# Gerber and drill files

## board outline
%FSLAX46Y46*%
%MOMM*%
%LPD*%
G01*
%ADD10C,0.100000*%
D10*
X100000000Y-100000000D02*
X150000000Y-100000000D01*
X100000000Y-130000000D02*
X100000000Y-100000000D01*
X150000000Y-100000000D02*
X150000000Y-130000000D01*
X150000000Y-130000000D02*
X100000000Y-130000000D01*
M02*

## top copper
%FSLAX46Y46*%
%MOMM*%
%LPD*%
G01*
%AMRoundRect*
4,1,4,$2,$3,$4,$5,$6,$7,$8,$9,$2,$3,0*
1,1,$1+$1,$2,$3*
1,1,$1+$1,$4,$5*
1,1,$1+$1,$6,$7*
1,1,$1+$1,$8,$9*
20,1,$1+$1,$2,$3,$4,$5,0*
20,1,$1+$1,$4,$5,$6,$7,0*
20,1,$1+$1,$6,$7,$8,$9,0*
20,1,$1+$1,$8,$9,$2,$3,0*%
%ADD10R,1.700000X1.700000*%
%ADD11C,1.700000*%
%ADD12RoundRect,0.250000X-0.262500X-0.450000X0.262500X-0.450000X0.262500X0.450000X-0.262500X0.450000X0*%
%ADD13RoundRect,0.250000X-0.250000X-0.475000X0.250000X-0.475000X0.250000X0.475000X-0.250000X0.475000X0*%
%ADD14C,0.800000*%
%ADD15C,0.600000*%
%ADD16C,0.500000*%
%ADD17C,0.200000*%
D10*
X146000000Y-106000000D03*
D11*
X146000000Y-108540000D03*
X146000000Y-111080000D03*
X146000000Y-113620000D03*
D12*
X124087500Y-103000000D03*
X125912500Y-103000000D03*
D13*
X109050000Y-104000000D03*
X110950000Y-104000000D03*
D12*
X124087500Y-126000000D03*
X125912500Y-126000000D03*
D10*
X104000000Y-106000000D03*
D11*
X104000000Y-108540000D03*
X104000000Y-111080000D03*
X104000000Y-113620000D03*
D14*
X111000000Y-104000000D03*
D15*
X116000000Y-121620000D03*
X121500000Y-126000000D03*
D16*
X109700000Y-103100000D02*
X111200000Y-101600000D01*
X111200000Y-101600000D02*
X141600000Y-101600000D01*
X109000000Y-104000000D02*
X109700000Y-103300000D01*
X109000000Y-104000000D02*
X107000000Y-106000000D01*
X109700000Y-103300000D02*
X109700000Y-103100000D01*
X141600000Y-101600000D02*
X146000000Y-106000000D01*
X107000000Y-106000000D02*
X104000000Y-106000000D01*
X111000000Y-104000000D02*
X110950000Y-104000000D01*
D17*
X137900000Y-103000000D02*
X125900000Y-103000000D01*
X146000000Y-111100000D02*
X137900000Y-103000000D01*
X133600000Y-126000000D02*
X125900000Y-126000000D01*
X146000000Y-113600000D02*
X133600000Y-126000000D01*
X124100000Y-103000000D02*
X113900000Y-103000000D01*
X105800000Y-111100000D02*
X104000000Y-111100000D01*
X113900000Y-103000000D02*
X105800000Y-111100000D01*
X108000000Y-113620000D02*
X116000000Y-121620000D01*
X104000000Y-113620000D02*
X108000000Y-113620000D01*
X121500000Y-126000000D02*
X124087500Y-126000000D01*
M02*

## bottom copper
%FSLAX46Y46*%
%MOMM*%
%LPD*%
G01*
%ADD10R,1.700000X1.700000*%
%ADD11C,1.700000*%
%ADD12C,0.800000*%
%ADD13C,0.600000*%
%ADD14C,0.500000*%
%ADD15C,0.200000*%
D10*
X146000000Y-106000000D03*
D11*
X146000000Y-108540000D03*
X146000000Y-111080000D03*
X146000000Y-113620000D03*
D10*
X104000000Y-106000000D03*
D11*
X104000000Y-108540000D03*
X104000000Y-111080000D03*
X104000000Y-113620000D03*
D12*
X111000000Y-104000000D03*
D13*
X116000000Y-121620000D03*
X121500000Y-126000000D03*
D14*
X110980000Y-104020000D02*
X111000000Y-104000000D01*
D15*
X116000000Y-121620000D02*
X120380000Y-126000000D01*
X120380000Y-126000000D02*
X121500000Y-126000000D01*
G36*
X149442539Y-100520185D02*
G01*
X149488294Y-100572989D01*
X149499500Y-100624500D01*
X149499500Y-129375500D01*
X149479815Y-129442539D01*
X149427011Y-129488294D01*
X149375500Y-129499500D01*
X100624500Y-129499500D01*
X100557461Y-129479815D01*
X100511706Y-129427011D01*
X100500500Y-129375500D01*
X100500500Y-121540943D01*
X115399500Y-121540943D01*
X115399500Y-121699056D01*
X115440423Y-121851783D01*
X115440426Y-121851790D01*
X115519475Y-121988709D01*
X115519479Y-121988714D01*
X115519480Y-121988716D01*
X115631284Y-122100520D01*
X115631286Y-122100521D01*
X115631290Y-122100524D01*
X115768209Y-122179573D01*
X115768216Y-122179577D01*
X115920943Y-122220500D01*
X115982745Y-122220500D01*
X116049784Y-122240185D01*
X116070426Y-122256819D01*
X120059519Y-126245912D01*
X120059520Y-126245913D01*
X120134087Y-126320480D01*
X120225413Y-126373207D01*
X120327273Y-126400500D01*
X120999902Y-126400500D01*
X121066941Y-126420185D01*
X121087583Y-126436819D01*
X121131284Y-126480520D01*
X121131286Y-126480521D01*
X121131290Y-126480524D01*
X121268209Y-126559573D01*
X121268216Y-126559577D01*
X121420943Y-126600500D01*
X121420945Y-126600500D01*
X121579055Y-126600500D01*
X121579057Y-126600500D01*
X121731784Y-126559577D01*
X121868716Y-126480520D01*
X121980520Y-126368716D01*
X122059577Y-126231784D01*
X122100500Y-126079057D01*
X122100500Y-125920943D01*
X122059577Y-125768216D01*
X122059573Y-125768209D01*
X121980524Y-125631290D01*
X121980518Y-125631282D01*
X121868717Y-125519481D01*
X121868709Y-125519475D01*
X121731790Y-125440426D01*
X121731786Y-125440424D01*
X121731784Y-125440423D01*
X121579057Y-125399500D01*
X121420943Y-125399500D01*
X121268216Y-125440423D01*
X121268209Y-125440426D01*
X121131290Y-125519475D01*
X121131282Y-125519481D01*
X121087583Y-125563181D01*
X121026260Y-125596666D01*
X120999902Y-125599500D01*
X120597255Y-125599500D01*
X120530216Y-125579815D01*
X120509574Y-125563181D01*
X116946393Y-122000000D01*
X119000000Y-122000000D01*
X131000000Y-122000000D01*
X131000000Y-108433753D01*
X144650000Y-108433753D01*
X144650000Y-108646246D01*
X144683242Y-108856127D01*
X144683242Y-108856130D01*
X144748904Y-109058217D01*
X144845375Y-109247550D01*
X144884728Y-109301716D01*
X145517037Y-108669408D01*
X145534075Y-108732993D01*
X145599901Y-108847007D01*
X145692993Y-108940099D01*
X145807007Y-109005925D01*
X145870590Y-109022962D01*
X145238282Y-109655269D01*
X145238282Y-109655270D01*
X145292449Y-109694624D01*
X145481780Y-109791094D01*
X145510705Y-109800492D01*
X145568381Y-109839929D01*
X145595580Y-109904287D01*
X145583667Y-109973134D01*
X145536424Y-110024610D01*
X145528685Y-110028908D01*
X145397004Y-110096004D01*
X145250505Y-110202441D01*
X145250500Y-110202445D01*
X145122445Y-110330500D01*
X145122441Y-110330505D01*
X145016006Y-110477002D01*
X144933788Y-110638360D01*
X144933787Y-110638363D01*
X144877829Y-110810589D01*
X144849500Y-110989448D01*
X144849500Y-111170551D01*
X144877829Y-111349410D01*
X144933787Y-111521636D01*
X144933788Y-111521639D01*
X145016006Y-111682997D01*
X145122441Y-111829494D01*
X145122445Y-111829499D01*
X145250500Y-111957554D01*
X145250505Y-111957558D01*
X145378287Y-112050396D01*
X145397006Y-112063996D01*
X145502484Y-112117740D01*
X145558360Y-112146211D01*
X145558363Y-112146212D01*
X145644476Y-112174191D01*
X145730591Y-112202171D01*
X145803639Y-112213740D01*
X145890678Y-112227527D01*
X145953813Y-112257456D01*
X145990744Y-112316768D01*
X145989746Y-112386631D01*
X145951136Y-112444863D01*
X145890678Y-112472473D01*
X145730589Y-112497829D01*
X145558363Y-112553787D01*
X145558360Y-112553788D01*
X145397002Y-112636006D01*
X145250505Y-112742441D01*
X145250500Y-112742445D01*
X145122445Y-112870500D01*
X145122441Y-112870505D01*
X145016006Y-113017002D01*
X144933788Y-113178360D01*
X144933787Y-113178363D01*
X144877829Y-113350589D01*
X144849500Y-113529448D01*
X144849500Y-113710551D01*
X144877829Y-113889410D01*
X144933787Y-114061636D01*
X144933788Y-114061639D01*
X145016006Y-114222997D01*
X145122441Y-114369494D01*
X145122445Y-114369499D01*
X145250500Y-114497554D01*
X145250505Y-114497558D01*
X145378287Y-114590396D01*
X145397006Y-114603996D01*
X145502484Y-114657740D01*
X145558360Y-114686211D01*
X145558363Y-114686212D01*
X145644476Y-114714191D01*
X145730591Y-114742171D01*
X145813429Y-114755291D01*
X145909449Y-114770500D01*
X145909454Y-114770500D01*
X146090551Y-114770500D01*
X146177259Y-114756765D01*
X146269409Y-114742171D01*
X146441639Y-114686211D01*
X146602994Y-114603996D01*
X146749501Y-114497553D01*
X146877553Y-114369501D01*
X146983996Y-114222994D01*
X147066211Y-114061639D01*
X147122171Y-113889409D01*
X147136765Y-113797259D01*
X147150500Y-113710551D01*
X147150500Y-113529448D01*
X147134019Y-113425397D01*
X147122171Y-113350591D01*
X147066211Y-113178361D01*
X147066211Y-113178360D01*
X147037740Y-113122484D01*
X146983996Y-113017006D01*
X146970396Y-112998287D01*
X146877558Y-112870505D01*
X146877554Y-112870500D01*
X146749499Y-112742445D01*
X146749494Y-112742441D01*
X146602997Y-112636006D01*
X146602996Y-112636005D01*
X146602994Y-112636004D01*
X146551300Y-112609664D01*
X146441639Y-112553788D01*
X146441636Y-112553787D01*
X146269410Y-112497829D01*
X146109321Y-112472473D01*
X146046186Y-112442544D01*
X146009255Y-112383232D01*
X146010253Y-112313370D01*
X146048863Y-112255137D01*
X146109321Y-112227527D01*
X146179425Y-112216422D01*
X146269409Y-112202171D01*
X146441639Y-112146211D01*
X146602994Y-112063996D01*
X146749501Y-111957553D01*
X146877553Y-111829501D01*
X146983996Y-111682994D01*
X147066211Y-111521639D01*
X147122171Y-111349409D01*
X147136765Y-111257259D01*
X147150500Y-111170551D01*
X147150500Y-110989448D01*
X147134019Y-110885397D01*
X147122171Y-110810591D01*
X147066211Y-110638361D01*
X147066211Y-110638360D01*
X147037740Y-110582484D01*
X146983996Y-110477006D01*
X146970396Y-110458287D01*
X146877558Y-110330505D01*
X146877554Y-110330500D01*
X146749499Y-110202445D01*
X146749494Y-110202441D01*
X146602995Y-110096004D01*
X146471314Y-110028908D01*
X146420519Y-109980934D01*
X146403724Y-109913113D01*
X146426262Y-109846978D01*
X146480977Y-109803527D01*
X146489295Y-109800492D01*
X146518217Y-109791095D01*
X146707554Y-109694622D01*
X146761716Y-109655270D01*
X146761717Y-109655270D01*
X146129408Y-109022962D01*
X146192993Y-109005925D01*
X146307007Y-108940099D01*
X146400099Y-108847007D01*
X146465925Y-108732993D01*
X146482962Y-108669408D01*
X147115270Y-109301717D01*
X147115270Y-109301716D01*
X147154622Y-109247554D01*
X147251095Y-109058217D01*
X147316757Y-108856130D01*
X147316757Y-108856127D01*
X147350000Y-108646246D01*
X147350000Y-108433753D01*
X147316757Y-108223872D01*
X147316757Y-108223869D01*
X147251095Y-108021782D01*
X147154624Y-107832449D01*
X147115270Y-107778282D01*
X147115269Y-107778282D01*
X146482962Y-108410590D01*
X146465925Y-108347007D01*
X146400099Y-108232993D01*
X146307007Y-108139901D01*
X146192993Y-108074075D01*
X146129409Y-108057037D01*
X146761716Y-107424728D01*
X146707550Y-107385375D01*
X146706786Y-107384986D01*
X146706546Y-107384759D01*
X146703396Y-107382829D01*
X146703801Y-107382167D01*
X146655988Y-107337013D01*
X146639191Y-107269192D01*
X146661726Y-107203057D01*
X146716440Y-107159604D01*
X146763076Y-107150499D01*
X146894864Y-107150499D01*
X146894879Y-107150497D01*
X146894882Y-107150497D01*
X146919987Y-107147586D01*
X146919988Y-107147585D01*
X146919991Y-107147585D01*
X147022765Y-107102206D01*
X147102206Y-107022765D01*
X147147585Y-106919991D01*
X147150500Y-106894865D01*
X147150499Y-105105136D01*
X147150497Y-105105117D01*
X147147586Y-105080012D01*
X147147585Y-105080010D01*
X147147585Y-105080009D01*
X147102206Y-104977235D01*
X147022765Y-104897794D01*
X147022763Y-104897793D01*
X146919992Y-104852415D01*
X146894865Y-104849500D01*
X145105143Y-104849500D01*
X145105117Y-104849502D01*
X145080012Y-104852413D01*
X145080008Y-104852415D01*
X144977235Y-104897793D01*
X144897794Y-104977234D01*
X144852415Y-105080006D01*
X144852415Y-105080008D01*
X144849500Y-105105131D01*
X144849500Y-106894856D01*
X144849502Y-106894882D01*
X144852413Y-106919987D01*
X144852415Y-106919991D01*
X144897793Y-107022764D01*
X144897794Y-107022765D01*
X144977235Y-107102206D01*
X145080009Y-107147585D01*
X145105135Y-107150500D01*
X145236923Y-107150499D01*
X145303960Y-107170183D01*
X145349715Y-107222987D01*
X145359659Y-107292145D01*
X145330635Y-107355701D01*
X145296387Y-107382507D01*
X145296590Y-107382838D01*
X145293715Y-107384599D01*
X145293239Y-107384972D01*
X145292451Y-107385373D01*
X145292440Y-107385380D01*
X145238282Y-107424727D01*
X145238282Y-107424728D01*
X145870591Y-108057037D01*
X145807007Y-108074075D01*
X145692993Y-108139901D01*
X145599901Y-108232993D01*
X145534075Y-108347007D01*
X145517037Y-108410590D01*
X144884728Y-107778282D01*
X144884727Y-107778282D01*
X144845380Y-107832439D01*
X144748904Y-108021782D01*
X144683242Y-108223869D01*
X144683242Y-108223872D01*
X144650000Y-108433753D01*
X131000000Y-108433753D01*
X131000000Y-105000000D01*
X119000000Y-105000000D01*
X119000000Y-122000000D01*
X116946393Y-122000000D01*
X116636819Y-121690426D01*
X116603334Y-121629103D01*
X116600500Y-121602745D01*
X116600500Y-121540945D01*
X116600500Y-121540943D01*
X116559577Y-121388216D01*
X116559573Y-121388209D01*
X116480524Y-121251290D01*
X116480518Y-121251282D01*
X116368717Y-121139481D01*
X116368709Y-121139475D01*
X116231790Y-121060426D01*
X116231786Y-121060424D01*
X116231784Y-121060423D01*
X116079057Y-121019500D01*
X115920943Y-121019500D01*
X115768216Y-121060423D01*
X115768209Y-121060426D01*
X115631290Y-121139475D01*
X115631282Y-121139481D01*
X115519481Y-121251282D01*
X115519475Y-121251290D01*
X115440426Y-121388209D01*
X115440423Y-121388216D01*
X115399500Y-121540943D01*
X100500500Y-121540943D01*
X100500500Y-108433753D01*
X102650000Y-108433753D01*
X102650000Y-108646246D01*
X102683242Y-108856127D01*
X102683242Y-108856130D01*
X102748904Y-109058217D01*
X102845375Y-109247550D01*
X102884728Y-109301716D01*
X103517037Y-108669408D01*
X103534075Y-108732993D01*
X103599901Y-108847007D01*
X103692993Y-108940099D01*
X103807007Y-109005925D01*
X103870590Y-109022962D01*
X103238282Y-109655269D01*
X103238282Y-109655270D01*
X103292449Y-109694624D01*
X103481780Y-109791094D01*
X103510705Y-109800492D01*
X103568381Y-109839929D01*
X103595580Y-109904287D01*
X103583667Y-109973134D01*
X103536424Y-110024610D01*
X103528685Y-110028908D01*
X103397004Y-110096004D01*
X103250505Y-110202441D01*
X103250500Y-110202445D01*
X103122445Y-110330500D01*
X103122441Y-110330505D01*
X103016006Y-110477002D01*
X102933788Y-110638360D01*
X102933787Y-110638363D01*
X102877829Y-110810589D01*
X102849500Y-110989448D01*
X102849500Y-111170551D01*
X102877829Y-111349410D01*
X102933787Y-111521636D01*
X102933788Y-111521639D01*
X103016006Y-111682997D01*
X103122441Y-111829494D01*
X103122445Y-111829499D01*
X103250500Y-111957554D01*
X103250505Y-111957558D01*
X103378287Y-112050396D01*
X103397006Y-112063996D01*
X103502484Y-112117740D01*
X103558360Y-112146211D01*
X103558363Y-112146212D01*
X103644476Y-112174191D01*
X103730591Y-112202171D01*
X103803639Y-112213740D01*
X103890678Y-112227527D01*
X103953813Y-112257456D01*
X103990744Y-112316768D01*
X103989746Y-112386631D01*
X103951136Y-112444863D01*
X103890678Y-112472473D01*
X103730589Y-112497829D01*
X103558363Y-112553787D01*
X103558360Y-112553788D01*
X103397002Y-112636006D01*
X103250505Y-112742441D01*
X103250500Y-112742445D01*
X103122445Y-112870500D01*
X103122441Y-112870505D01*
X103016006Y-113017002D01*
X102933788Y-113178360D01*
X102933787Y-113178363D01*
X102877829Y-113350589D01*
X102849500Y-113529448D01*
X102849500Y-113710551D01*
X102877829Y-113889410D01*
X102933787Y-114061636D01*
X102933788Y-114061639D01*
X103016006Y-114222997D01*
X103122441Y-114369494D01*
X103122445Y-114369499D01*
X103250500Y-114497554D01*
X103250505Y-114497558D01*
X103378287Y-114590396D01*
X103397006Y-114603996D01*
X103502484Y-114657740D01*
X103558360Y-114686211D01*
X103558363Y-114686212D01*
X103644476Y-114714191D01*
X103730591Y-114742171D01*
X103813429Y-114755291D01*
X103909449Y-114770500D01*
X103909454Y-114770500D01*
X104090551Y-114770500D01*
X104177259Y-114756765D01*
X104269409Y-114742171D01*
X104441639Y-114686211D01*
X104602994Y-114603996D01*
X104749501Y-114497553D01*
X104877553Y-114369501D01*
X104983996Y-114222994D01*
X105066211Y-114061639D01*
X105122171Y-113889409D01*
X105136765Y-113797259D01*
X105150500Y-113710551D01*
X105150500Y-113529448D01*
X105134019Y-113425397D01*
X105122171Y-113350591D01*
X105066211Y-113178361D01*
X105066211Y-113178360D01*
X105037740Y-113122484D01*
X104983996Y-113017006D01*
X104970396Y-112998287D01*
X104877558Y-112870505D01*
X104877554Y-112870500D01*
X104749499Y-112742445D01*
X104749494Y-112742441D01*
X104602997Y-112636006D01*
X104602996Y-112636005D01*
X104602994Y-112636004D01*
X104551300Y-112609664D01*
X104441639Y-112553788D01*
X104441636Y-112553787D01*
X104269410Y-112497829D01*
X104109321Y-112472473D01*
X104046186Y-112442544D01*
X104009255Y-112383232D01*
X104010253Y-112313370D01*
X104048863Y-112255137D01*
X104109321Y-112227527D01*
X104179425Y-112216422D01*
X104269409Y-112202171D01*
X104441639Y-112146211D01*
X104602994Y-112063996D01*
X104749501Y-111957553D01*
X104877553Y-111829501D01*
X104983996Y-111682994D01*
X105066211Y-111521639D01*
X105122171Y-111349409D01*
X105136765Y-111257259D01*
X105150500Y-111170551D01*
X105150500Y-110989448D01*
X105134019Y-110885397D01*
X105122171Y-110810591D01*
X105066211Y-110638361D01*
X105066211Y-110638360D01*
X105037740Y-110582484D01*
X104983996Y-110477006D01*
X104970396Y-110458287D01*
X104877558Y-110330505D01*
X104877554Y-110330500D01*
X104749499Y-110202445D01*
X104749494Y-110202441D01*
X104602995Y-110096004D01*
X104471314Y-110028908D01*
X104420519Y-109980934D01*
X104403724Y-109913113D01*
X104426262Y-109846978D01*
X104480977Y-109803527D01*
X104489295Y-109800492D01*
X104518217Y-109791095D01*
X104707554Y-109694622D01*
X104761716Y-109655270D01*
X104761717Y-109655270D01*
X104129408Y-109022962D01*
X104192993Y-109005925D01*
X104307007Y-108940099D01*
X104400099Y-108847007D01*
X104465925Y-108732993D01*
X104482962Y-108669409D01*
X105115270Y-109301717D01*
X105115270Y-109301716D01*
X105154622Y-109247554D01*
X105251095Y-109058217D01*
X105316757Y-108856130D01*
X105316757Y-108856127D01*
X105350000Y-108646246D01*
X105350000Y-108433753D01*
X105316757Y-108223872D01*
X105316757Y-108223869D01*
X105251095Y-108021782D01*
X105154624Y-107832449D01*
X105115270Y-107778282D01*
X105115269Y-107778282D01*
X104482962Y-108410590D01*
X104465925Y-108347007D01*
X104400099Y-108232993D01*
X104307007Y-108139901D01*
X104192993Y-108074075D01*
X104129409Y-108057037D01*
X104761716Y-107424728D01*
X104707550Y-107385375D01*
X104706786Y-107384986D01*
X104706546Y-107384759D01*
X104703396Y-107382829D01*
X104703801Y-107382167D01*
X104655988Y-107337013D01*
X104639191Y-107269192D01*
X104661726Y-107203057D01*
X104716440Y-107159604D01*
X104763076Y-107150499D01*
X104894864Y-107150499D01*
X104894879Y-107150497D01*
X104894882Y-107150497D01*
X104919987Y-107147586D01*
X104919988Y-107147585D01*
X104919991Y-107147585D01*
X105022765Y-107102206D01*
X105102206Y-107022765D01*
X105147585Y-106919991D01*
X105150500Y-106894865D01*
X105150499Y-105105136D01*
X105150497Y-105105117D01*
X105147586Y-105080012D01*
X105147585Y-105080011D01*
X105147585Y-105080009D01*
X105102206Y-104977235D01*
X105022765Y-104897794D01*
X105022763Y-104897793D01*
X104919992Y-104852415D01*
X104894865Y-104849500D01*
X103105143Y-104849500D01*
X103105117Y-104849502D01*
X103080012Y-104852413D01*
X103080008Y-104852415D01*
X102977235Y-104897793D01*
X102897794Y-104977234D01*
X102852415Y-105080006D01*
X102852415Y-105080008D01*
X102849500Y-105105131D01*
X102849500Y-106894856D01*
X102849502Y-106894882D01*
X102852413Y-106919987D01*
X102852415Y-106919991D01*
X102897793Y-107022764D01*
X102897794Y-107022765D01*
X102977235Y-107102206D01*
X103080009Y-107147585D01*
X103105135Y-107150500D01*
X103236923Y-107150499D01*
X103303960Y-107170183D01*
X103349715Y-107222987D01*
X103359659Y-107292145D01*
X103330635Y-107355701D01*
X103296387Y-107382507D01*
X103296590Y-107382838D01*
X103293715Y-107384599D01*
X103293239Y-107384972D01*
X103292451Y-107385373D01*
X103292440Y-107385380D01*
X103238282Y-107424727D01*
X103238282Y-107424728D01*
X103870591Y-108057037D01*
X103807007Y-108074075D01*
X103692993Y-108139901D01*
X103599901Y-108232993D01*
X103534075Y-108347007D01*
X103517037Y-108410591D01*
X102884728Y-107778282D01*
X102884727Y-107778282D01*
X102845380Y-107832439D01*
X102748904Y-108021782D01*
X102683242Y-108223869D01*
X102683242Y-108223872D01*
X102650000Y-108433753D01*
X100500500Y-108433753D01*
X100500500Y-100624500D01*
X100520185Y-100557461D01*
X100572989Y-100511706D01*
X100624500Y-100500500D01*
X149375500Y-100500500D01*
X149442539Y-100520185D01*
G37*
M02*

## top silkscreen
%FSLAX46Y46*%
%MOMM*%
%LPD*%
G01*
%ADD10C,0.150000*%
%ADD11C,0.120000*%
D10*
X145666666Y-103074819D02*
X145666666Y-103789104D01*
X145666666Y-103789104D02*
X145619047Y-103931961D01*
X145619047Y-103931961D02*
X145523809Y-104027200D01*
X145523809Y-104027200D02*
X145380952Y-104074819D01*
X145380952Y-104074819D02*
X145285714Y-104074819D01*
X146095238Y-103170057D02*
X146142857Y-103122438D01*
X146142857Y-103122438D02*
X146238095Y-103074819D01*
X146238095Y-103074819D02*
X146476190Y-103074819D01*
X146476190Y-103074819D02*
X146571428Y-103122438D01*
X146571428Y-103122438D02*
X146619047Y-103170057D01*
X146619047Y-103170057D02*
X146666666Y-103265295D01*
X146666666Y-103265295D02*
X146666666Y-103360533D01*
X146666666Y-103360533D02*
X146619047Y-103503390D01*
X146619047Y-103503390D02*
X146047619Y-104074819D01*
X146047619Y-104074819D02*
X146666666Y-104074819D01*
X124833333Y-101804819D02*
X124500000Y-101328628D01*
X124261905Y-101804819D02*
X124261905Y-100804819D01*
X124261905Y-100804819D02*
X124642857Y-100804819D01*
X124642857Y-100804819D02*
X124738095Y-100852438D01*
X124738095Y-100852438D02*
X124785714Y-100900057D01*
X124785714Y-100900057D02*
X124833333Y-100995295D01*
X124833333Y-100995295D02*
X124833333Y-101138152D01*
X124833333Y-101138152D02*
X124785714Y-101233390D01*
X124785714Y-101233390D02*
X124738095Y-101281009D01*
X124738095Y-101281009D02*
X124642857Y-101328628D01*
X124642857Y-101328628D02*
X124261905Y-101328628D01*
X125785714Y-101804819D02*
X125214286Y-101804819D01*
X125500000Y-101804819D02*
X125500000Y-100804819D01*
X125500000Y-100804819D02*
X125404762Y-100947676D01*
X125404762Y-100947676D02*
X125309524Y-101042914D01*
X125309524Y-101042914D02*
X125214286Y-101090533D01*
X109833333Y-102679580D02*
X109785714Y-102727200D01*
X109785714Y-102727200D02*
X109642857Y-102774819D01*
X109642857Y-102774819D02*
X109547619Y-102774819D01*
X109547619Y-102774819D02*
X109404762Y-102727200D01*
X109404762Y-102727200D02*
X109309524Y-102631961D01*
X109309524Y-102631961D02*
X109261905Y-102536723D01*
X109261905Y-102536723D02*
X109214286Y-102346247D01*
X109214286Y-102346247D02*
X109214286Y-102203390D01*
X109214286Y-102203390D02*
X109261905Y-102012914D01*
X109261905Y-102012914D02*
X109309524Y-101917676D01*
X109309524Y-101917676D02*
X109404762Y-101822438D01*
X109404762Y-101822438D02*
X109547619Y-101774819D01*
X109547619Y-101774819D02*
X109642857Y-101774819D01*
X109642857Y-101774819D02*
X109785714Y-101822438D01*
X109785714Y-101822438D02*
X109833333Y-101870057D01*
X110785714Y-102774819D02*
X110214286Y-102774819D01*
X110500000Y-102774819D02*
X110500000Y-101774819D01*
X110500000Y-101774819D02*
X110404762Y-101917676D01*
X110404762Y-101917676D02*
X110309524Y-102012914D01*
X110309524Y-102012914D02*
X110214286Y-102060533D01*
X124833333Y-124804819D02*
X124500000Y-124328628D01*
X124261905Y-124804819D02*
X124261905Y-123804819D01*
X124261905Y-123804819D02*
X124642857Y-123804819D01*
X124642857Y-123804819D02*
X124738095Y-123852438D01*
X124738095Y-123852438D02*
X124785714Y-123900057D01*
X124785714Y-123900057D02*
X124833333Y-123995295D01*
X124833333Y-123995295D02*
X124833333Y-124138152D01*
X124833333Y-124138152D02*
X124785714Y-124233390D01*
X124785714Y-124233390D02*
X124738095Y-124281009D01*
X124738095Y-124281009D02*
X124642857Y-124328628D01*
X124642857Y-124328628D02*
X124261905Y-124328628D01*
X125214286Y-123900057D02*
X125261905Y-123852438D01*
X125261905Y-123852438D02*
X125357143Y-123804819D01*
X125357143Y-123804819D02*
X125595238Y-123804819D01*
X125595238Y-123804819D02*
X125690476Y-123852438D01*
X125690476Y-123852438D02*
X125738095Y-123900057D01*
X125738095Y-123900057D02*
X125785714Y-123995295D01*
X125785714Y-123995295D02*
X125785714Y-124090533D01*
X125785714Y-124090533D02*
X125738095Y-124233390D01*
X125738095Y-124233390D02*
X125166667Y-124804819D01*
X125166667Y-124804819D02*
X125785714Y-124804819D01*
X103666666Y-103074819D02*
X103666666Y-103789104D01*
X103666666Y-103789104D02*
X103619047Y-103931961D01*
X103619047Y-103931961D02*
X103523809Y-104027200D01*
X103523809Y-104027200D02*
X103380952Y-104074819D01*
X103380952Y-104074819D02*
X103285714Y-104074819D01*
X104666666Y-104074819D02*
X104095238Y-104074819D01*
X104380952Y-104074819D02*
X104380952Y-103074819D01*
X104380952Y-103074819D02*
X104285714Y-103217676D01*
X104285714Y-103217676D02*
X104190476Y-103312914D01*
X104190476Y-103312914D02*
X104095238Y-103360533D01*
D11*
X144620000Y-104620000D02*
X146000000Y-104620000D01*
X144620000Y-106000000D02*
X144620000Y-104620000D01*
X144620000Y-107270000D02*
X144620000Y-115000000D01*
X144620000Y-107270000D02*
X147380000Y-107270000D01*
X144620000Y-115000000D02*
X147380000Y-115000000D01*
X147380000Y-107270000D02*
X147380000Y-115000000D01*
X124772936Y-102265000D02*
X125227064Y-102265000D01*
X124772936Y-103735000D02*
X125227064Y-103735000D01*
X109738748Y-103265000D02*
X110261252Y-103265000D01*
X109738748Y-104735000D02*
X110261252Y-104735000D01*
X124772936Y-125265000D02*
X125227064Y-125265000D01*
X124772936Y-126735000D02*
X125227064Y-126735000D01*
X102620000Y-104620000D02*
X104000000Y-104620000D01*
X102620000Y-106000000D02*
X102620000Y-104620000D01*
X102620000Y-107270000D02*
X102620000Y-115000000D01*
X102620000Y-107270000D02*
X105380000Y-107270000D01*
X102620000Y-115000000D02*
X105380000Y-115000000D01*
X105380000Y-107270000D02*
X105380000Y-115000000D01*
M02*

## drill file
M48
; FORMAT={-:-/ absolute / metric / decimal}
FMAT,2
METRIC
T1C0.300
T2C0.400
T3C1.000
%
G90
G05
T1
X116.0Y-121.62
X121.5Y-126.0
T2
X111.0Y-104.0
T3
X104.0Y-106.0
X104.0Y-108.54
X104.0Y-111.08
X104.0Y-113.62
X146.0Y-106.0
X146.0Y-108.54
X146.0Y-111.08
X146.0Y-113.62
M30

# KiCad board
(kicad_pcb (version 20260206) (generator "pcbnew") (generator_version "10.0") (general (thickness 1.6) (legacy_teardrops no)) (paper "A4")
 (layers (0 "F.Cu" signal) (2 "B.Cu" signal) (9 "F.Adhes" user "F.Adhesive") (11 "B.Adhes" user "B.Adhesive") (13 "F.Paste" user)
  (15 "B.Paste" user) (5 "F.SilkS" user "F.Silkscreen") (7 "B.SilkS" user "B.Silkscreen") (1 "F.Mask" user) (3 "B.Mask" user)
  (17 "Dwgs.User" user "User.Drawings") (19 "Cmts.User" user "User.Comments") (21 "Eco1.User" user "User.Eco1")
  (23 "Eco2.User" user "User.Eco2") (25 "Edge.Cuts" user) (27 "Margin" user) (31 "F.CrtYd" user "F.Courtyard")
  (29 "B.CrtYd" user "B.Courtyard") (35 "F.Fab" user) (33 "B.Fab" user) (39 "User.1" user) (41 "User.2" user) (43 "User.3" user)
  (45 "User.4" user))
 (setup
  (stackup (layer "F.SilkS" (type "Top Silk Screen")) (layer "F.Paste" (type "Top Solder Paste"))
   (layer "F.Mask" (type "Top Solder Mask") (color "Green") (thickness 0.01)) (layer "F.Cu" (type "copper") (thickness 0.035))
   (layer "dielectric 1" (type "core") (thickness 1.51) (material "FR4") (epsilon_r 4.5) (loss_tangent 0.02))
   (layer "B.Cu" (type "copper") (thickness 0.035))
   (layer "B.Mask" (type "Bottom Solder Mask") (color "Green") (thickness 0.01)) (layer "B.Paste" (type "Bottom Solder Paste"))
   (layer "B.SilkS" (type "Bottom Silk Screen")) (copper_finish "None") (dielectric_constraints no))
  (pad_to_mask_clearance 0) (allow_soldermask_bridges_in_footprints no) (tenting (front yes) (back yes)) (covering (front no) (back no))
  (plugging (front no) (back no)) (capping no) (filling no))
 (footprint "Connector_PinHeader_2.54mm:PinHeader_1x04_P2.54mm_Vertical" (layer "F.Cu") (at 146 106)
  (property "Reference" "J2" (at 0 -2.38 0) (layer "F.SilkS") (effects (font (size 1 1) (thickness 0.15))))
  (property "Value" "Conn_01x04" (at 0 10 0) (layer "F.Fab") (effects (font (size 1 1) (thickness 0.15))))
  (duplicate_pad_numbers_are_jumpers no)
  (fp_line (start -1.38 -1.38) (end 0 -1.38) (stroke (width 0.12) (type solid)) (layer "F.SilkS"))
  (fp_line (start -1.38 0) (end -1.38 -1.38) (stroke (width 0.12) (type solid)) (layer "F.SilkS"))
  (fp_line (start -1.38 1.27) (end -1.38 9) (stroke (width 0.12) (type solid)) (layer "F.SilkS"))
  (fp_line (start -1.38 1.27) (end 1.38 1.27) (stroke (width 0.12) (type solid)) (layer "F.SilkS"))
  (fp_line (start -1.38 9) (end 1.38 9) (stroke (width 0.12) (type solid)) (layer "F.SilkS"))
  (fp_line (start 1.38 1.27) (end 1.38 9) (stroke (width 0.12) (type solid)) (layer "F.SilkS"))
  (pad "1" thru_hole rect (at 0 0) (size 1.7 1.7) (drill 1) (layers "*.Cu" "*.Mask") (remove_unused_layers no) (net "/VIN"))
  (pad "2" thru_hole circle (at 0 2.54) (size 1.7 1.7) (drill 1) (layers "*.Cu" "*.Mask") (remove_unused_layers no) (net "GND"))
  (pad "3" thru_hole circle (at 0 5.08) (size 1.7 1.7) (drill 1) (layers "*.Cu" "*.Mask") (remove_unused_layers no) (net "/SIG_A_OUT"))
  (pad "4" thru_hole circle (at 0 7.62) (size 1.7 1.7) (drill 1) (layers "*.Cu" "*.Mask") (remove_unused_layers no) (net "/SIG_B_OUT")))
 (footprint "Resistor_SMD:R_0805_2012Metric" (layer "F.Cu") (at 125 103)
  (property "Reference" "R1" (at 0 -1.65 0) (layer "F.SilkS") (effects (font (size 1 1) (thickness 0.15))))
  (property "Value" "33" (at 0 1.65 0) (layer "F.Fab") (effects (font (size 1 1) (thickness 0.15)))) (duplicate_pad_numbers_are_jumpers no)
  (fp_line (start -0.227064 -0.735) (end 0.227064 -0.735) (stroke (width 0.12) (type solid)) (layer "F.SilkS"))
  (fp_line (start -0.227064 0.735) (end 0.227064 0.735) (stroke (width 0.12) (type solid)) (layer "F.SilkS"))
  (pad "1" smd roundrect (at -0.9125 0) (size 1.025 1.4) (layers "F.Cu" "F.Mask" "F.Paste") (roundrect_rratio 0.243902) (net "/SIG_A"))
  (pad "2" smd roundrect (at 0.9125 0) (size 1.025 1.4) (layers "F.Cu" "F.Mask" "F.Paste") (roundrect_rratio 0.243902) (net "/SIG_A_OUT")))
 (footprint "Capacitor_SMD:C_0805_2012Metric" (layer "F.Cu") (at 110 104)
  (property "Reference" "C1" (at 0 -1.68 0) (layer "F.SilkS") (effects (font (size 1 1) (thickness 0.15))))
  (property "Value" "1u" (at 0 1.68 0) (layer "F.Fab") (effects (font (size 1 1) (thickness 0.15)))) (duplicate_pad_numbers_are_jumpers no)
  (fp_line (start -0.261252 -0.735) (end 0.261252 -0.735) (stroke (width 0.12) (type solid)) (layer "F.SilkS"))
  (fp_line (start -0.261252 0.735) (end 0.261252 0.735) (stroke (width 0.12) (type solid)) (layer "F.SilkS"))
  (pad "1" smd roundrect (at -0.95 0) (size 1 1.45) (layers "F.Cu" "F.Mask" "F.Paste") (roundrect_rratio 0.25) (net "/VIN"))
  (pad "2" smd roundrect (at 0.95 0) (size 1 1.45) (layers "F.Cu" "F.Mask" "F.Paste") (roundrect_rratio 0.25) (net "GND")))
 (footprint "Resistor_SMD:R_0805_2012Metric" (layer "F.Cu") (at 125 126)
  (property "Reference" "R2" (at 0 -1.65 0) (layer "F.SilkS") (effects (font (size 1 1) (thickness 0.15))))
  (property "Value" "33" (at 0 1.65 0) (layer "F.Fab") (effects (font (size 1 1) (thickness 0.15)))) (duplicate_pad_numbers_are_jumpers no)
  (fp_line (start -0.227064 -0.735) (end 0.227064 -0.735) (stroke (width 0.12) (type solid)) (layer "F.SilkS"))
  (fp_line (start -0.227064 0.735) (end 0.227064 0.735) (stroke (width 0.12) (type solid)) (layer "F.SilkS"))
  (pad "1" smd roundrect (at -0.9125 0) (size 1.025 1.4) (layers "F.Cu" "F.Mask" "F.Paste") (roundrect_rratio 0.243902) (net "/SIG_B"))
  (pad "2" smd roundrect (at 0.9125 0) (size 1.025 1.4) (layers "F.Cu" "F.Mask" "F.Paste") (roundrect_rratio 0.243902) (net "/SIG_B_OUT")))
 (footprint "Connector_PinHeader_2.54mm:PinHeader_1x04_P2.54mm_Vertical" (layer "F.Cu") (at 104 106)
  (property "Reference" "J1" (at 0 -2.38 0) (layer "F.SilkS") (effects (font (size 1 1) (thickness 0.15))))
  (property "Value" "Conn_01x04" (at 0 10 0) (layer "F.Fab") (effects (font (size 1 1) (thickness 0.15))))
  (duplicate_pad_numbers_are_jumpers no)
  (fp_line (start -1.38 -1.38) (end 0 -1.38) (stroke (width 0.12) (type solid)) (layer "F.SilkS"))
  (fp_line (start -1.38 0) (end -1.38 -1.38) (stroke (width 0.12) (type solid)) (layer "F.SilkS"))
  (fp_line (start -1.38 1.27) (end -1.38 9) (stroke (width 0.12) (type solid)) (layer "F.SilkS"))
  (fp_line (start -1.38 1.27) (end 1.38 1.27) (stroke (width 0.12) (type solid)) (layer "F.SilkS"))
  (fp_line (start -1.38 9) (end 1.38 9) (stroke (width 0.12) (type solid)) (layer "F.SilkS"))
  (fp_line (start 1.38 1.27) (end 1.38 9) (stroke (width 0.12) (type solid)) (layer "F.SilkS"))
  (pad "1" thru_hole rect (at 0 0) (size 1.7 1.7) (drill 1) (layers "*.Cu" "*.Mask") (remove_unused_layers no) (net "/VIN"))
  (pad "2" thru_hole circle (at 0 2.54) (size 1.7 1.7) (drill 1) (layers "*.Cu" "*.Mask") (remove_unused_layers no) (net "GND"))
  (pad "3" thru_hole circle (at 0 5.08) (size 1.7 1.7) (drill 1) (layers "*.Cu" "*.Mask") (remove_unused_layers no) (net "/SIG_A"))
  (pad "4" thru_hole circle (at 0 7.62) (size 1.7 1.7) (drill 1) (layers "*.Cu" "*.Mask") (remove_unused_layers no) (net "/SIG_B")))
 (gr_line (start 100 100) (end 150 100) (stroke (width 0.1) (type default)) (layer "Edge.Cuts"))
 (gr_line (start 100 130) (end 100 100) (stroke (width 0.1) (type default)) (layer "Edge.Cuts"))
 (gr_line (start 150 100) (end 150 130) (stroke (width 0.1) (type default)) (layer "Edge.Cuts"))
 (gr_line (start 150 130) (end 100 130) (stroke (width 0.1) (type default)) (layer "Edge.Cuts"))
 (segment (start 109.7 103.1) (end 111.2 101.6) (width 0.5) (layer "F.Cu") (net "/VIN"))
 (segment (start 111.2 101.6) (end 141.6 101.6) (width 0.5) (layer "F.Cu") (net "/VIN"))
 (segment (start 109 104) (end 109.7 103.3) (width 0.5) (layer "F.Cu") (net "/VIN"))
 (segment (start 109 104) (end 107 106) (width 0.5) (layer "F.Cu") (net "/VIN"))
 (segment (start 109.7 103.3) (end 109.7 103.1) (width 0.5) (layer "F.Cu") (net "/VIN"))
 (segment (start 141.6 101.6) (end 146 106) (width 0.5) (layer "F.Cu") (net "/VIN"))
 (segment (start 107 106) (end 104 106) (width 0.5) (layer "F.Cu") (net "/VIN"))
 (segment (start 111 104) (end 110.95 104) (width 0.5) (layer "F.Cu") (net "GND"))
 (via (at 111 104) (size 0.8) (drill 0.4) (layers "F.Cu" "B.Cu") (capping yes) (filling yes) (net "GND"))
 (segment (start 110.98 104.02) (end 111 104) (width 0.5) (layer "B.Cu") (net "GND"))
 (segment (start 137.9 103) (end 125.9 103) (width 0.2) (layer "F.Cu") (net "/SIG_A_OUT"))
 (segment (start 146 111.1) (end 137.9 103) (width 0.2) (layer "F.Cu") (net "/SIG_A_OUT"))
 (segment (start 133.6 126) (end 125.9 126) (width 0.2) (layer "F.Cu") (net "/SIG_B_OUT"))
 (segment (start 146 113.6) (end 133.6 126) (width 0.2) (layer "F.Cu") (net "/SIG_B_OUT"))
 (segment (start 124.1 103) (end 113.9 103) (width 0.2) (layer "F.Cu") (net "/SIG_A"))
 (segment (start 105.8 111.1) (end 104 111.1) (width 0.2) (layer "F.Cu") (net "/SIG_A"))
 (segment (start 113.9 103) (end 105.8 111.1) (width 0.2) (layer "F.Cu") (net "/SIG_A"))
 (segment (start 108 113.62) (end 116 121.62) (width 0.2) (locked yes) (layer "F.Cu") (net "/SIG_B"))
 (segment (start 104 113.62) (end 108 113.62) (width 0.2) (locked yes) (layer "F.Cu") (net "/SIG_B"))
 (segment (start 121.5 126) (end 124.0875 126) (width 0.2) (locked yes) (layer "F.Cu") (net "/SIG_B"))
 (via (at 116 121.62) (size 0.6) (drill 0.3) (layers "F.Cu" "B.Cu") (locked yes) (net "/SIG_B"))
 (via (at 121.5 126) (size 0.6) (drill 0.3) (layers "F.Cu" "B.Cu") (locked yes) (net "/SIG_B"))
 (segment (start 116 121.62) (end 120.38 126) (width 0.2) (locked yes) (layer "B.Cu") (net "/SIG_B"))
 (segment (start 120.38 126) (end 121.5 126) (width 0.2) (locked yes) (layer "B.Cu") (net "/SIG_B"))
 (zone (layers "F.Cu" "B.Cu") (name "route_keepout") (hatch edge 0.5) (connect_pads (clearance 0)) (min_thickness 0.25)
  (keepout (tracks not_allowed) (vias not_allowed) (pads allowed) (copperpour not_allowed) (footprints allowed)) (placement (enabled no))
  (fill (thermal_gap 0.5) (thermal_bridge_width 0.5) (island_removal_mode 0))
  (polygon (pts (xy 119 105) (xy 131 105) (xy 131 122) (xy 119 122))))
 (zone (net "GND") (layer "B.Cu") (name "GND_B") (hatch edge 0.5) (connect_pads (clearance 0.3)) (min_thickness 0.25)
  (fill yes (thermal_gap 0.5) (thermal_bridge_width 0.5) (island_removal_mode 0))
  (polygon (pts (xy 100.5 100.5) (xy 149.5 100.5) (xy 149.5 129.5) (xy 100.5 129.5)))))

